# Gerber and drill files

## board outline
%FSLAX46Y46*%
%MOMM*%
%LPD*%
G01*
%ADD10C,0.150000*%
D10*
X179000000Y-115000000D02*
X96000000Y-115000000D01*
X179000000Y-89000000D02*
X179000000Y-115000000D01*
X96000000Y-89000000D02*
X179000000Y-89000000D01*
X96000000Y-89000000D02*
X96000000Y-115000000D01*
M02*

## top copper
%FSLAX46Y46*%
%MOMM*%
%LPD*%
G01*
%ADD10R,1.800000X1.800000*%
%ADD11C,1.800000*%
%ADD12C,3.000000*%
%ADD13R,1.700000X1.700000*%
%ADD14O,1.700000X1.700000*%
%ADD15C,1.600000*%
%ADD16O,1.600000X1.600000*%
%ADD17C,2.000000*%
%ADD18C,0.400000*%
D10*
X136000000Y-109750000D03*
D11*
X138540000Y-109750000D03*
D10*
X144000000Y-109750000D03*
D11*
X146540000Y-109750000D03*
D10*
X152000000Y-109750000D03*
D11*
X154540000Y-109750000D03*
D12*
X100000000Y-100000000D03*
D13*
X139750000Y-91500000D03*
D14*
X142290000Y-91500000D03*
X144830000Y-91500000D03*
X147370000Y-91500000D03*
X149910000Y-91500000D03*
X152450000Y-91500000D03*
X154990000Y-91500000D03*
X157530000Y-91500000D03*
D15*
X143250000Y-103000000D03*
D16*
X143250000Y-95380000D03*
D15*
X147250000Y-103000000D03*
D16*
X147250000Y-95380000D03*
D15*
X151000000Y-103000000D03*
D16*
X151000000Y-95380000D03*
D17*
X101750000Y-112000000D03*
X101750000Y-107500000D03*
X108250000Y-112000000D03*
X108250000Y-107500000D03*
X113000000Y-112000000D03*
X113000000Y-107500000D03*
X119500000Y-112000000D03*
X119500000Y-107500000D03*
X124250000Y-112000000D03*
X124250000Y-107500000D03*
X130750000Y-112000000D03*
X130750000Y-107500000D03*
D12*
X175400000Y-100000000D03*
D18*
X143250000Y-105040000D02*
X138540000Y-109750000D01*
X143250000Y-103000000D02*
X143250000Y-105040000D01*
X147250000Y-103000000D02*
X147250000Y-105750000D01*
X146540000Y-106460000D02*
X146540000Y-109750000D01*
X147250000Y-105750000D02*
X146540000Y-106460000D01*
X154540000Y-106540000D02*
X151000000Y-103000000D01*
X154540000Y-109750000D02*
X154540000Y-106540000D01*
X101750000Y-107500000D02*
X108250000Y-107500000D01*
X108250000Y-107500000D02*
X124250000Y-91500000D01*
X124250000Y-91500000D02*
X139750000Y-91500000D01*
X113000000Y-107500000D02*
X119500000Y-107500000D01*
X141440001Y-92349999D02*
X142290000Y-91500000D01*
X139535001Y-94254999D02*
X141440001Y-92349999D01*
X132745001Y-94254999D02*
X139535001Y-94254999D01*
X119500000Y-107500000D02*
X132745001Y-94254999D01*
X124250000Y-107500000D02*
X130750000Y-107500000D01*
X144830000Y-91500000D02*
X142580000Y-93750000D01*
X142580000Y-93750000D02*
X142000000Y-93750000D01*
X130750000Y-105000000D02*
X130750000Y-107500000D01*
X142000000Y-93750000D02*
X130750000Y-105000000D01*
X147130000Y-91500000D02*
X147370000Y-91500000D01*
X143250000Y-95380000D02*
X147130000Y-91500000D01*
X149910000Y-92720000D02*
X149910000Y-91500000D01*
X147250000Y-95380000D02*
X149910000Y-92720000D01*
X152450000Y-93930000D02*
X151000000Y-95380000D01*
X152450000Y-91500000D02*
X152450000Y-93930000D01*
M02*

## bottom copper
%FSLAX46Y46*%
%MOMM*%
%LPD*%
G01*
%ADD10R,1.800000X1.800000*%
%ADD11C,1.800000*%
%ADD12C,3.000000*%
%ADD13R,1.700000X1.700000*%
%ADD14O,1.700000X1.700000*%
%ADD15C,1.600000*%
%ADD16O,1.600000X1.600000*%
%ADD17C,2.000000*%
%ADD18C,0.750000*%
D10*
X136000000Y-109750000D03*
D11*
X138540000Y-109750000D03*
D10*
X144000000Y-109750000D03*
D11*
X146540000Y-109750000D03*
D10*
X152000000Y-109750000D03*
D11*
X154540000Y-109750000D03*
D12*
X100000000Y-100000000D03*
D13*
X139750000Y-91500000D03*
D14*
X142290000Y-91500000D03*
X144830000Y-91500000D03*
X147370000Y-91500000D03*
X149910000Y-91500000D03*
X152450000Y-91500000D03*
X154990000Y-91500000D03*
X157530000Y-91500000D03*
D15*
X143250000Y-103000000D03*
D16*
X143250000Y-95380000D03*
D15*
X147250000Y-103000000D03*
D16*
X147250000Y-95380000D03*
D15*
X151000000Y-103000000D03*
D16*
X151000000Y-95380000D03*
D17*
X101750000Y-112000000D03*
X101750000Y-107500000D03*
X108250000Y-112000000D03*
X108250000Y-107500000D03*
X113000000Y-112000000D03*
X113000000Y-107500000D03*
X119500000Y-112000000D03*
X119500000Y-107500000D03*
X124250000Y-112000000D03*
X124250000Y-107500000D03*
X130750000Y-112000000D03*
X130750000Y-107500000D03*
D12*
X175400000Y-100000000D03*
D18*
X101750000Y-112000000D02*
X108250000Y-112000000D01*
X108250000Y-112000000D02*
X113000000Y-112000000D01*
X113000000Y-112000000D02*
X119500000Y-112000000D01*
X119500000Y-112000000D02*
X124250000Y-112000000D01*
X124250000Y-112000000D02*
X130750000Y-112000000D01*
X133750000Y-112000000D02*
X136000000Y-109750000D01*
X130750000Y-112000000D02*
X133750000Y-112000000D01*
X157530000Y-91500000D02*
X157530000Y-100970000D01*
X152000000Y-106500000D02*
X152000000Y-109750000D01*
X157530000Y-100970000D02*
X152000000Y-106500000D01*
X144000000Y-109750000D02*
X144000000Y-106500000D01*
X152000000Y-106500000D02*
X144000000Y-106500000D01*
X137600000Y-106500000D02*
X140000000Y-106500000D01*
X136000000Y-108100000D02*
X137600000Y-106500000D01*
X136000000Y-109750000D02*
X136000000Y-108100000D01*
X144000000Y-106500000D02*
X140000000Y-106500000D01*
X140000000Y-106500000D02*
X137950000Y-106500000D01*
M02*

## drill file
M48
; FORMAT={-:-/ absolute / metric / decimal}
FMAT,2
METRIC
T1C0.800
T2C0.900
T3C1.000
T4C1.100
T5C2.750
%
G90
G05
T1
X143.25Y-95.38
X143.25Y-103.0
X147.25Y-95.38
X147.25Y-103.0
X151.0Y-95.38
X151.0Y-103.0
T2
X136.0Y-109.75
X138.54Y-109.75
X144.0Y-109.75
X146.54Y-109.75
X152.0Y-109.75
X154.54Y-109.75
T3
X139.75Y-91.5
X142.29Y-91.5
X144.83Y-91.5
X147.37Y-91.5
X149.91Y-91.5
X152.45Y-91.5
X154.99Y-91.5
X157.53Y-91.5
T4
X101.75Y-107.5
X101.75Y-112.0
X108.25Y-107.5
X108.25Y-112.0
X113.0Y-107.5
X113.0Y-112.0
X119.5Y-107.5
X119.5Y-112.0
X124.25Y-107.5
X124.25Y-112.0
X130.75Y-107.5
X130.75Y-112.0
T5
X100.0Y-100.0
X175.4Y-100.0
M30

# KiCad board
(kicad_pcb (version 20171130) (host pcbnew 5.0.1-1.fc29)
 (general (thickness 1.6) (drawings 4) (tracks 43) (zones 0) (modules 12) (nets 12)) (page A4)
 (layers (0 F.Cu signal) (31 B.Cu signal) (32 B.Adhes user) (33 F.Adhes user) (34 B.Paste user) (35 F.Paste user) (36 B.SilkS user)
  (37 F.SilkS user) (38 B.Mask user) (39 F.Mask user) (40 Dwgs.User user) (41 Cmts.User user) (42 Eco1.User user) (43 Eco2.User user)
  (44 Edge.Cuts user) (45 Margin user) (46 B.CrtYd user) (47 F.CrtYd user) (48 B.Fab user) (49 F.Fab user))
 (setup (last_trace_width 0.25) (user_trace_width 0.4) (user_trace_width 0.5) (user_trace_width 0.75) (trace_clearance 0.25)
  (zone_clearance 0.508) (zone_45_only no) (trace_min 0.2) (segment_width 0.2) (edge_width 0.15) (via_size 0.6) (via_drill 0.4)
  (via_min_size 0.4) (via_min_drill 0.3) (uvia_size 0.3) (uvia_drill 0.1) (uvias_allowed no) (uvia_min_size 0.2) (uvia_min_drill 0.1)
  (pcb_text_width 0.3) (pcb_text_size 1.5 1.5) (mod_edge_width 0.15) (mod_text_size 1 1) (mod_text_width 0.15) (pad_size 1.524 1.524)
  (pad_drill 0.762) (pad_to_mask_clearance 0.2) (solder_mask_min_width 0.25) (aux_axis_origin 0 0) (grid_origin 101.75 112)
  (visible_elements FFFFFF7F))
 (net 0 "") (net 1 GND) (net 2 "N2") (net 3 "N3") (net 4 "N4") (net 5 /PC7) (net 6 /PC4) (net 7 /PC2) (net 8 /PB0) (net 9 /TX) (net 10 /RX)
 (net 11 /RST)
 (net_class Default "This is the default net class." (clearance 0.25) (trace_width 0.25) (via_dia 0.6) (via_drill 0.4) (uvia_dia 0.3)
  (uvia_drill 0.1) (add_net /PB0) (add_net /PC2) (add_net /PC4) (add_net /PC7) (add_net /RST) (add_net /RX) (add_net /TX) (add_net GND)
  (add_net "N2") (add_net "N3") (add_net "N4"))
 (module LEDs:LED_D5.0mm (layer F.Cu) (at 136 109.75)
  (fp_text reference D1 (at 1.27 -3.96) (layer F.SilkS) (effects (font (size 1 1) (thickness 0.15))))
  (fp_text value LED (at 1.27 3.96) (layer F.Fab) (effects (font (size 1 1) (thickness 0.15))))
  (pad 1 thru_hole rect (at 0 0) (size 1.8 1.8) (drill 0.9) (layers *.Cu *.Mask) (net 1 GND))
  (pad 2 thru_hole circle (at 2.54 0) (size 1.8 1.8) (drill 0.9) (layers *.Cu *.Mask) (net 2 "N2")))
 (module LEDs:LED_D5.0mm (layer F.Cu) (at 144 109.75)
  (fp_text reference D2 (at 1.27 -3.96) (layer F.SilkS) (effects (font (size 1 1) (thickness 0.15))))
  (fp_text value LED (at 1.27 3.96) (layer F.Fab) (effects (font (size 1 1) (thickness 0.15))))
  (pad 1 thru_hole rect (at 0 0) (size 1.8 1.8) (drill 0.9) (layers *.Cu *.Mask) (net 1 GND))
  (pad 2 thru_hole circle (at 2.54 0) (size 1.8 1.8) (drill 0.9) (layers *.Cu *.Mask) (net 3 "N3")))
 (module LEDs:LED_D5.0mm (layer F.Cu) (at 152 109.75)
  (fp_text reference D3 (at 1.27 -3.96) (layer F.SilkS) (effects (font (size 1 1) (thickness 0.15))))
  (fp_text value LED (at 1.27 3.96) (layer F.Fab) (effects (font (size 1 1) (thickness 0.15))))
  (pad 1 thru_hole rect (at 0 0) (size 1.8 1.8) (drill 0.9) (layers *.Cu *.Mask) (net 1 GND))
  (pad 2 thru_hole circle (at 2.54 0) (size 1.8 1.8) (drill 0.9) (layers *.Cu *.Mask) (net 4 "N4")))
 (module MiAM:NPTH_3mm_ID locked (layer F.Cu) (at 100 100)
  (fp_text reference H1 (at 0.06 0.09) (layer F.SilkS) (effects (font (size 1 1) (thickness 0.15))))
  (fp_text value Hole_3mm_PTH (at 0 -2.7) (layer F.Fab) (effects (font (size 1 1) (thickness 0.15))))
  (pad "" np_thru_hole circle (at 0 0) (size 3 3) (drill 2.75) (layers *.Cu *.Mask) (clearance 1.6)))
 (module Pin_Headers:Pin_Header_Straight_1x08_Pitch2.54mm (layer F.Cu) (at 139.75 91.5 90)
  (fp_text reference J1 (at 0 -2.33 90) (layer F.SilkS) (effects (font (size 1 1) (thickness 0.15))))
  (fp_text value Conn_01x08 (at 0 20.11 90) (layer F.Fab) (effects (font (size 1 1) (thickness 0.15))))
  (pad 1 thru_hole rect (at 0 0 90) (size 1.7 1.7) (drill 1) (layers *.Cu *.Mask) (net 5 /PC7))
  (pad 2 thru_hole oval (at 0 2.54 90) (size 1.7 1.7) (drill 1) (layers *.Cu *.Mask) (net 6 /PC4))
  (pad 3 thru_hole oval (at 0 5.08 90) (size 1.7 1.7) (drill 1) (layers *.Cu *.Mask) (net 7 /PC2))
  (pad 4 thru_hole oval (at 0 7.62 90) (size 1.7 1.7) (drill 1) (layers *.Cu *.Mask) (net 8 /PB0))
  (pad 5 thru_hole oval (at 0 10.16 90) (size 1.7 1.7) (drill 1) (layers *.Cu *.Mask) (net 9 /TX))
  (pad 6 thru_hole oval (at 0 12.7 90) (size 1.7 1.7) (drill 1) (layers *.Cu *.Mask) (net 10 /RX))
  (pad 7 thru_hole oval (at 0 15.24 90) (size 1.7 1.7) (drill 1) (layers *.Cu *.Mask) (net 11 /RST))
  (pad 8 thru_hole oval (at 0 17.78 90) (size 1.7 1.7) (drill 1) (layers *.Cu *.Mask) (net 1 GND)))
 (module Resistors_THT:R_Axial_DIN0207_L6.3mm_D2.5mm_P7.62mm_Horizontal (layer F.Cu) (at 143.25 103 90)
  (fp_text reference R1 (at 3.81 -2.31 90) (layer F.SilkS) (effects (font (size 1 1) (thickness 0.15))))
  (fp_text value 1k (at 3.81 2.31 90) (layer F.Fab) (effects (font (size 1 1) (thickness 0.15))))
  (pad 1 thru_hole circle (at 0 0 90) (size 1.6 1.6) (drill 0.8) (layers *.Cu *.Mask) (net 2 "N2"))
  (pad 2 thru_hole oval (at 7.62 0 90) (size 1.6 1.6) (drill 0.8) (layers *.Cu *.Mask) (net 8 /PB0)))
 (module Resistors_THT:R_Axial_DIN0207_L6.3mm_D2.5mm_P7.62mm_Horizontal (layer F.Cu) (at 147.25 103 90)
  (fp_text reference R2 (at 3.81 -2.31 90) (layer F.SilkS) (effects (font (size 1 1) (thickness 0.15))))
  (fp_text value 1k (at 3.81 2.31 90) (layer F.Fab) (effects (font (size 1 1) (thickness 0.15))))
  (pad 1 thru_hole circle (at 0 0 90) (size 1.6 1.6) (drill 0.8) (layers *.Cu *.Mask) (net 3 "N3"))
  (pad 2 thru_hole oval (at 7.62 0 90) (size 1.6 1.6) (drill 0.8) (layers *.Cu *.Mask) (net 9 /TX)))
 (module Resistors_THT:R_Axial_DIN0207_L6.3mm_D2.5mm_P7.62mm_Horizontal (layer F.Cu) (at 151 103 90)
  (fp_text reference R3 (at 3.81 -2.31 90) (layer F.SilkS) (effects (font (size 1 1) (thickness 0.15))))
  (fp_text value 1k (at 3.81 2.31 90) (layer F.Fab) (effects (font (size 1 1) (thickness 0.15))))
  (pad 1 thru_hole circle (at 0 0 90) (size 1.6 1.6) (drill 0.8) (layers *.Cu *.Mask) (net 4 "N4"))
  (pad 2 thru_hole oval (at 7.62 0 90) (size 1.6 1.6) (drill 0.8) (layers *.Cu *.Mask) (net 10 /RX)))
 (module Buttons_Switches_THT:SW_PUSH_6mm (layer F.Cu) (at 101.75 107.5)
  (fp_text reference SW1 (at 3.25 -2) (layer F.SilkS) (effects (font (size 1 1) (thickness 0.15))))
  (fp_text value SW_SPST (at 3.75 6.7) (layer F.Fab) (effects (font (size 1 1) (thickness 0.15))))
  (pad 2 thru_hole circle (at 0 4.5 90) (size 2 2) (drill 1.1) (layers *.Cu *.Mask) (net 1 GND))
  (pad 1 thru_hole circle (at 0 0 90) (size 2 2) (drill 1.1) (layers *.Cu *.Mask) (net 5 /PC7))
  (pad 2 thru_hole circle (at 6.5 4.5 90) (size 2 2) (drill 1.1) (layers *.Cu *.Mask) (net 1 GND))
  (pad 1 thru_hole circle (at 6.5 0 90) (size 2 2) (drill 1.1) (layers *.Cu *.Mask) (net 5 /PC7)))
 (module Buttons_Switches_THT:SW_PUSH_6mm (layer F.Cu) (at 113 107.5)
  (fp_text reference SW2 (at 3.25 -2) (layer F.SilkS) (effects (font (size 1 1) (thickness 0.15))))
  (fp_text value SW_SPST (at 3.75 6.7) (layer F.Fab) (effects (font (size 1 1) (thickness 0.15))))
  (pad 2 thru_hole circle (at 0 4.5 90) (size 2 2) (drill 1.1) (layers *.Cu *.Mask) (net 1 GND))
  (pad 1 thru_hole circle (at 0 0 90) (size 2 2) (drill 1.1) (layers *.Cu *.Mask) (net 6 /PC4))
  (pad 2 thru_hole circle (at 6.5 4.5 90) (size 2 2) (drill 1.1) (layers *.Cu *.Mask) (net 1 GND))
  (pad 1 thru_hole circle (at 6.5 0 90) (size 2 2) (drill 1.1) (layers *.Cu *.Mask) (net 6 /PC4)))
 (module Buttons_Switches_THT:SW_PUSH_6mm (layer F.Cu) (at 124.25 107.5)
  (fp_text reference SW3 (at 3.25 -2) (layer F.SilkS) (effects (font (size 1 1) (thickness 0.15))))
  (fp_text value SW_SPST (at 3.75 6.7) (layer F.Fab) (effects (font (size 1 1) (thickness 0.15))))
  (pad 2 thru_hole circle (at 0 4.5 90) (size 2 2) (drill 1.1) (layers *.Cu *.Mask) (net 1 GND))
  (pad 1 thru_hole circle (at 0 0 90) (size 2 2) (drill 1.1) (layers *.Cu *.Mask) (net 7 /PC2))
  (pad 2 thru_hole circle (at 6.5 4.5 90) (size 2 2) (drill 1.1) (layers *.Cu *.Mask) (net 1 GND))
  (pad 1 thru_hole circle (at 6.5 0 90) (size 2 2) (drill 1.1) (layers *.Cu *.Mask) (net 7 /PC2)))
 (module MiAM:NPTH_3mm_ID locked (layer F.Cu) (at 175.4 100)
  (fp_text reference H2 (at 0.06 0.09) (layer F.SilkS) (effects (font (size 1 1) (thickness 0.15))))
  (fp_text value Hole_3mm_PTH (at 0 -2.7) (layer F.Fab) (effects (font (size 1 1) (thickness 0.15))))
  (pad "" np_thru_hole circle (at 0 0) (size 3 3) (drill 2.75) (layers *.Cu *.Mask) (clearance 1.6)))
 (gr_line (start 179 115) (end 96 115) (angle 90) (layer Edge.Cuts) (width 0.15))
 (gr_line (start 179 89) (end 179 115) (angle 90) (layer Edge.Cuts) (width 0.15))
 (gr_line (start 96 89) (end 179 89) (angle 90) (layer Edge.Cuts) (width 0.15))
 (gr_line (start 96 89) (end 96 115) (angle 90) (layer Edge.Cuts) (width 0.15))
 (segment (start 101.75 112) (end 108.25 112) (width 0.75) (layer B.Cu) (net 1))
 (segment (start 108.25 112) (end 113 112) (width 0.75) (layer B.Cu) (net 1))
 (segment (start 113 112) (end 119.5 112) (width 0.75) (layer B.Cu) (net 1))
 (segment (start 119.5 112) (end 124.25 112) (width 0.75) (layer B.Cu) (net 1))
 (segment (start 124.25 112) (end 130.75 112) (width 0.75) (layer B.Cu) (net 1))
 (segment (start 133.75 112) (end 136 109.75) (width 0.75) (layer B.Cu) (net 1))
 (segment (start 130.75 112) (end 133.75 112) (width 0.75) (layer B.Cu) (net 1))
 (segment (start 157.53 91.5) (end 157.53 100.97) (width 0.75) (layer B.Cu) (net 1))
 (segment (start 152 106.5) (end 152 109.75) (width 0.75) (layer B.Cu) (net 1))
 (segment (start 157.53 100.97) (end 152 106.5) (width 0.75) (layer B.Cu) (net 1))
 (segment (start 144 109.75) (end 144 106.5) (width 0.75) (layer B.Cu) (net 1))
 (segment (start 152 106.5) (end 144 106.5) (width 0.75) (layer B.Cu) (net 1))
 (segment (start 137.6 106.5) (end 140 106.5) (width 0.75) (layer B.Cu) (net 1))
 (segment (start 136 108.1) (end 137.6 106.5) (width 0.75) (layer B.Cu) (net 1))
 (segment (start 136 109.75) (end 136 108.1) (width 0.75) (layer B.Cu) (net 1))
 (segment (start 144 106.5) (end 140 106.5) (width 0.75) (layer B.Cu) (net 1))
 (segment (start 140 106.5) (end 137.95 106.5) (width 0.75) (layer B.Cu) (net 1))
 (segment (start 143.25 105.04) (end 138.54 109.75) (width 0.4) (layer F.Cu) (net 2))
 (segment (start 143.25 103) (end 143.25 105.04) (width 0.4) (layer F.Cu) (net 2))
 (segment (start 147.25 103) (end 147.25 105.75) (width 0.4) (layer F.Cu) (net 3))
 (segment (start 146.54 106.46) (end 146.54 109.75) (width 0.4) (layer F.Cu) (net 3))
 (segment (start 147.25 105.75) (end 146.54 106.46) (width 0.4) (layer F.Cu) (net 3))
 (segment (start 154.54 106.54) (end 151 103) (width 0.4) (layer F.Cu) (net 4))
 (segment (start 154.54 109.75) (end 154.54 106.54) (width 0.4) (layer F.Cu) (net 4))
 (segment (start 101.75 107.5) (end 108.25 107.5) (width 0.4) (layer F.Cu) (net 5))
 (segment (start 108.25 107.5) (end 124.25 91.5) (width 0.4) (layer F.Cu) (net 5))
 (segment (start 124.25 91.5) (end 139.75 91.5) (width 0.4) (layer F.Cu) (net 5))
 (segment (start 113 107.5) (end 119.5 107.5) (width 0.4) (layer F.Cu) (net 6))
 (segment (start 141.440001 92.349999) (end 142.29 91.5) (width 0.4) (layer F.Cu) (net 6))
 (segment (start 139.535001 94.254999) (end 141.440001 92.349999) (width 0.4) (layer F.Cu) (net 6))
 (segment (start 132.745001 94.254999) (end 139.535001 94.254999) (width 0.4) (layer F.Cu) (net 6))
 (segment (start 119.5 107.5) (end 132.745001 94.254999) (width 0.4) (layer F.Cu) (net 6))
 (segment (start 124.25 107.5) (end 130.75 107.5) (width 0.4) (layer F.Cu) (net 7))
 (segment (start 144.83 91.5) (end 142.58 93.75) (width 0.4) (layer F.Cu) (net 7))
 (segment (start 142.58 93.75) (end 142 93.75) (width 0.4) (layer F.Cu) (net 7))
 (segment (start 130.75 105) (end 130.75 107.5) (width 0.4) (layer F.Cu) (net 7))
 (segment (start 142 93.75) (end 130.75 105) (width 0.4) (layer F.Cu) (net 7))
 (segment (start 147.13 91.5) (end 147.37 91.5) (width 0.4) (layer F.Cu) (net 8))
 (segment (start 143.25 95.38) (end 147.13 91.5) (width 0.4) (layer F.Cu) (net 8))
 (segment (start 149.91 92.72) (end 149.91 91.5) (width 0.4) (layer F.Cu) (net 9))
 (segment (start 147.25 95.38) (end 149.91 92.72) (width 0.4) (layer F.Cu) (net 9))
 (segment (start 152.45 93.93) (end 151 95.38) (width 0.4) (layer F.Cu) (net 10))
 (segment (start 152.45 91.5) (end 152.45 93.93) (width 0.4) (layer F.Cu) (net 10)))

